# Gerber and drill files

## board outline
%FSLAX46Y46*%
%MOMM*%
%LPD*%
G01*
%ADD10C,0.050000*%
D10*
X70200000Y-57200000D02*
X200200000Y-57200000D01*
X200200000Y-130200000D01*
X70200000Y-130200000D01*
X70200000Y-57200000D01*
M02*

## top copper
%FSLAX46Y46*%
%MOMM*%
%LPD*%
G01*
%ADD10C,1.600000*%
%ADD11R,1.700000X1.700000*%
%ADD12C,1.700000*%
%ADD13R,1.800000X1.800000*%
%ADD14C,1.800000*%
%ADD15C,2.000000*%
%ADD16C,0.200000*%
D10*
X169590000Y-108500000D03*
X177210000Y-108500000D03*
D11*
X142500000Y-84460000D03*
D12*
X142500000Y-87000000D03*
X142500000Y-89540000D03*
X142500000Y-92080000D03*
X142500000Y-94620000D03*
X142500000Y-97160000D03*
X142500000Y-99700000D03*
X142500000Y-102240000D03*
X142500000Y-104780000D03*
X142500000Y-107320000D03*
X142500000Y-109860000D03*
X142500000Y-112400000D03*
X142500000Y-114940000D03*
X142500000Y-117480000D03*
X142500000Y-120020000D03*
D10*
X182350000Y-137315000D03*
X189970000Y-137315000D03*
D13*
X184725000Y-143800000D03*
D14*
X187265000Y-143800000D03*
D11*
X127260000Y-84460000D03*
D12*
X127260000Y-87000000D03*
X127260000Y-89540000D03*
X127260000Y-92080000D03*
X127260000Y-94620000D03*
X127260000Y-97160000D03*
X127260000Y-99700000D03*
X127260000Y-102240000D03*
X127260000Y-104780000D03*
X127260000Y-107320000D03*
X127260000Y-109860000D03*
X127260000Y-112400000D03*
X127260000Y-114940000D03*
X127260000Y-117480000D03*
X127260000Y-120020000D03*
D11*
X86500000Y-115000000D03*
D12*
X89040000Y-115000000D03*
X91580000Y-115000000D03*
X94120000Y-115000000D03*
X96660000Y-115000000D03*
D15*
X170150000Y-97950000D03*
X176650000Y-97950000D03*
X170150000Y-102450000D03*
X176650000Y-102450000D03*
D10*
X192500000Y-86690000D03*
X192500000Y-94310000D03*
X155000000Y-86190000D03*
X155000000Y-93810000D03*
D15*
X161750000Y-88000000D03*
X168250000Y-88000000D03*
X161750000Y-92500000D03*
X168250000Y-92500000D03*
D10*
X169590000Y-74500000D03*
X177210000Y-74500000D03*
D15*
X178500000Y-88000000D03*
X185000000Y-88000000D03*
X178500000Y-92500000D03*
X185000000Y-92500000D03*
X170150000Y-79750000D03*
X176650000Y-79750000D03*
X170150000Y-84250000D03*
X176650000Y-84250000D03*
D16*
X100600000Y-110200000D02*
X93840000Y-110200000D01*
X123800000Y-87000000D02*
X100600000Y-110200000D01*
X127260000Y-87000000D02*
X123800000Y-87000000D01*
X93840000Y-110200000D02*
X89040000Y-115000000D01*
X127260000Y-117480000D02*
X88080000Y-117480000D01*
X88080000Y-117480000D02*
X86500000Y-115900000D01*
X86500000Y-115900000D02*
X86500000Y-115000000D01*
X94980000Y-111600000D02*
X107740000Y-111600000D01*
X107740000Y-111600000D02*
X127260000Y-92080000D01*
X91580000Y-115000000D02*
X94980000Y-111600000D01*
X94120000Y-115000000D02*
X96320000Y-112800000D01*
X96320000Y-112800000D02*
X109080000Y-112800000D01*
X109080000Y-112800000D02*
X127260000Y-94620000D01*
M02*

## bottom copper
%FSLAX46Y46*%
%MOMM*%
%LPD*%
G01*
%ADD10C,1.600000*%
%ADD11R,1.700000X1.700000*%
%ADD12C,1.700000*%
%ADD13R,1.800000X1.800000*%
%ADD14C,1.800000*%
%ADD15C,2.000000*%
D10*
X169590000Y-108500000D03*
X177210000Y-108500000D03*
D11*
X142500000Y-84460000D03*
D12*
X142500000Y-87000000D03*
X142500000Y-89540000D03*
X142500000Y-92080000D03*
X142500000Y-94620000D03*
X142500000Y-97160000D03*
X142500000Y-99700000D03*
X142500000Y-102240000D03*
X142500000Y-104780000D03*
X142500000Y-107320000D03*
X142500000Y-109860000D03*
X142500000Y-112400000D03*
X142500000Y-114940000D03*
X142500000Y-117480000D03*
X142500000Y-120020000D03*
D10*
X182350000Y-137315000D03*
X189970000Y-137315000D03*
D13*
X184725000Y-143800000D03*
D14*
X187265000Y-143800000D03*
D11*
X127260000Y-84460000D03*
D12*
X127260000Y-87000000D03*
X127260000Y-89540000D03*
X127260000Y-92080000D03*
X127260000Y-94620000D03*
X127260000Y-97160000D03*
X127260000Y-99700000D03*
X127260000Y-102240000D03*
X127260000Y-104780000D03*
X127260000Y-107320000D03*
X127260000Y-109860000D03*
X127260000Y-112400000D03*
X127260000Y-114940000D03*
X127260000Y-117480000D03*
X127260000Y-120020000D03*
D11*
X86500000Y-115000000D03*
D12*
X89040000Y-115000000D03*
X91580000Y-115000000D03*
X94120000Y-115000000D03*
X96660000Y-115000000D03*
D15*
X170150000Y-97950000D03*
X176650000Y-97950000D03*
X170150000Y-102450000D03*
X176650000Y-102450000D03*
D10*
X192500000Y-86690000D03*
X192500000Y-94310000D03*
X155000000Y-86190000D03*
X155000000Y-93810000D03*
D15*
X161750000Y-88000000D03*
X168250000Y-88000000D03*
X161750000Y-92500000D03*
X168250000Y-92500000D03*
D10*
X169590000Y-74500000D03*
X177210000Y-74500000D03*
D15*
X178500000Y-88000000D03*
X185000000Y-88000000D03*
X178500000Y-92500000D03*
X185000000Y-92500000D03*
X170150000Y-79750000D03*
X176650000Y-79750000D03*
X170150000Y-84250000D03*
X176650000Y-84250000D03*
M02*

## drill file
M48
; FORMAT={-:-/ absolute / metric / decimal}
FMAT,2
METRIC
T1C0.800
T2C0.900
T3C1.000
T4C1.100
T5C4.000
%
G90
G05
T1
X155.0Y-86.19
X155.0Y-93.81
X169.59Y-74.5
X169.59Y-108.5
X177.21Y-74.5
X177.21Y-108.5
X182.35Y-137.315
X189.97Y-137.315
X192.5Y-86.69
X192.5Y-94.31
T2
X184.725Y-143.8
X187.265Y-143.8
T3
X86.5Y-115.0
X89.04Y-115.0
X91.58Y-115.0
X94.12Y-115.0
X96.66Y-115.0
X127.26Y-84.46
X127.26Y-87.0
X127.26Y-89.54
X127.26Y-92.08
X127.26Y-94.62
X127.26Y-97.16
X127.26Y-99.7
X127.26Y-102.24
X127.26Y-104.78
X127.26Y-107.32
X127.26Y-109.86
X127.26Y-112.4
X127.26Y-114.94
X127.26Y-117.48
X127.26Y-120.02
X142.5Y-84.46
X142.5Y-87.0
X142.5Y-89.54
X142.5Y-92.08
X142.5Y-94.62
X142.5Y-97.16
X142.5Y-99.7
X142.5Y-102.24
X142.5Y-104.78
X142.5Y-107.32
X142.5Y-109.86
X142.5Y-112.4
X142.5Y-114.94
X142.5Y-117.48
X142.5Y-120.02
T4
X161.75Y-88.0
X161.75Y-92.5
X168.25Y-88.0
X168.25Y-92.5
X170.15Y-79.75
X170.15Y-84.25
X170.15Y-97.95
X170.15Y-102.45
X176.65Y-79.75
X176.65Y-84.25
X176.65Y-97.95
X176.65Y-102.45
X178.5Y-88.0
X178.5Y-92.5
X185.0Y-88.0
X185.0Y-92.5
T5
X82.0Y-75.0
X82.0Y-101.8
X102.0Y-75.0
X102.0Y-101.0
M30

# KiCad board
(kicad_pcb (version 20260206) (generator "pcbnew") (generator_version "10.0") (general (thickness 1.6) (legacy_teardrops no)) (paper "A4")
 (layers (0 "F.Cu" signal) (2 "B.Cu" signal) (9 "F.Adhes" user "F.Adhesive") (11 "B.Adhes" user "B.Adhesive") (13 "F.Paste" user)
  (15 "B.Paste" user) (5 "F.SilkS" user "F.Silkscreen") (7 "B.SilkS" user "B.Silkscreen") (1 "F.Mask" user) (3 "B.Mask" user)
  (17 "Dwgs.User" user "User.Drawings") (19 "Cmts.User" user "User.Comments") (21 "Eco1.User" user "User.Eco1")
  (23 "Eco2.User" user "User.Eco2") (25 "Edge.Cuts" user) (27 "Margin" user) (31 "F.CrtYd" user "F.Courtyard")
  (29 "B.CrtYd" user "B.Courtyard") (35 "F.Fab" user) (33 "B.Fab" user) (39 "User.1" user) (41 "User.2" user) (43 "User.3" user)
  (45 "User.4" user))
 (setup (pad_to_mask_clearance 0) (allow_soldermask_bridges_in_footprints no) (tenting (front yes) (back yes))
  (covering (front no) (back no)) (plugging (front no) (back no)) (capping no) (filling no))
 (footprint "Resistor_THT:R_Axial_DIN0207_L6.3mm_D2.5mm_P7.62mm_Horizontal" (layer "F.Cu") (at 169.59 108.5)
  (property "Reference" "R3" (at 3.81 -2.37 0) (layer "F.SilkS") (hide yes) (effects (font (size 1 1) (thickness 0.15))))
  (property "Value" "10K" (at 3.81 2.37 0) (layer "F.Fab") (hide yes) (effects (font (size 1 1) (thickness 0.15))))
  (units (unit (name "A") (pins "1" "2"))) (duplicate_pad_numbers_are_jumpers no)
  (pad "1" thru_hole circle (at 0 0) (size 1.6 1.6) (drill 0.8) (layers "*.Cu" "*.Mask") (remove_unused_layers no) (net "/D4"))
  (pad "2" thru_hole circle (at 7.62 0) (size 1.6 1.6) (drill 0.8) (layers "*.Cu" "*.Mask") (remove_unused_layers no) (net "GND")))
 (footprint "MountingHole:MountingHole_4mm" (layer "F.Cu") (at 102 75)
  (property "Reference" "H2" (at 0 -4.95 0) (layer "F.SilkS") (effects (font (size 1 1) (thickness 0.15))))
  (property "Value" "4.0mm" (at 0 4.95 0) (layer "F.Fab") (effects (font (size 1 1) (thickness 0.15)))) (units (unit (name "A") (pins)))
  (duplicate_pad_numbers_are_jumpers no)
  (pad "" np_thru_hole circle (at 0 0) (size 4 4) (drill 4) (layers "*.Cu" "*.Mask")))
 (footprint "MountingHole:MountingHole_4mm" (layer "F.Cu") (at 82 75)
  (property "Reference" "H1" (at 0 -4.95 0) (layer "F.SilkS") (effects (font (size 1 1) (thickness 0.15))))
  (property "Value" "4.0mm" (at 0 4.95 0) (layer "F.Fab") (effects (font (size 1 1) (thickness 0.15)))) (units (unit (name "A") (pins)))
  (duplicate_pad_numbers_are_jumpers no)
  (pad "" np_thru_hole circle (at 0 0) (size 4 4) (drill 4) (layers "*.Cu" "*.Mask")))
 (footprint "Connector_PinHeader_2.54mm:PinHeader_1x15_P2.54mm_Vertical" (layer "F.Cu") (at 142.5 84.46)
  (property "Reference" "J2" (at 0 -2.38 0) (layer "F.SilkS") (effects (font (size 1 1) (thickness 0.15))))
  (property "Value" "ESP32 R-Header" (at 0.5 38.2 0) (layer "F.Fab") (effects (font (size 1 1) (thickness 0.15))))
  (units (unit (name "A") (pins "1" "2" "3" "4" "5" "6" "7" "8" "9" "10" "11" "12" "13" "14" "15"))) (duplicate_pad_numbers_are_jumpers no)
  (pad "1" thru_hole rect (at 0 0) (size 1.7 1.7) (drill 1) (layers "*.Cu" "*.Mask") (remove_unused_layers no) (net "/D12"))
  (pad "2" thru_hole circle (at 0 2.54) (size 1.7 1.7) (drill 1) (layers "*.Cu" "*.Mask") (remove_unused_layers no) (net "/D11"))
  (pad "3" thru_hole circle (at 0 5.08) (size 1.7 1.7) (drill 1) (layers "*.Cu" "*.Mask") (remove_unused_layers no) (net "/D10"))
  (pad "4" thru_hole circle (at 0 7.62) (size 1.7 1.7) (drill 1) (layers "*.Cu" "*.Mask") (remove_unused_layers no) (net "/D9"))
  (pad "5" thru_hole circle (at 0 10.16) (size 1.7 1.7) (drill 1) (layers "*.Cu" "*.Mask") (remove_unused_layers no) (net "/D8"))
  (pad "6" thru_hole circle (at 0 12.7) (size 1.7 1.7) (drill 1) (layers "*.Cu" "*.Mask") (remove_unused_layers no) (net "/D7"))
  (pad "7" thru_hole circle (at 0 15.24) (size 1.7 1.7) (drill 1) (layers "*.Cu" "*.Mask") (remove_unused_layers no) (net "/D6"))
  (pad "8" thru_hole circle (at 0 17.78) (size 1.7 1.7) (drill 1) (layers "*.Cu" "*.Mask") (remove_unused_layers no) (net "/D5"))
  (pad "9" thru_hole circle (at 0 20.32) (size 1.7 1.7) (drill 1) (layers "*.Cu" "*.Mask") (remove_unused_layers no) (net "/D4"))
  (pad "10" thru_hole circle (at 0 22.86) (size 1.7 1.7) (drill 1) (layers "*.Cu" "*.Mask") (remove_unused_layers no) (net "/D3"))
  (pad "11" thru_hole circle (at 0 25.4) (size 1.7 1.7) (drill 1) (layers "*.Cu" "*.Mask") (remove_unused_layers no) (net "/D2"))
  (pad "12" thru_hole circle (at 0 27.94) (size 1.7 1.7) (drill 1) (layers "*.Cu" "*.Mask") (remove_unused_layers no) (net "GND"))
  (pad "13" thru_hole circle (at 0 30.48) (size 1.7 1.7) (drill 1) (layers "*.Cu" "*.Mask") (remove_unused_layers no) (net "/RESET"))
  (pad "14" thru_hole circle (at 0 33.02) (size 1.7 1.7) (drill 1) (layers "*.Cu" "*.Mask") (remove_unused_layers no) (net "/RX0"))
  (pad "15" thru_hole circle (at 0 35.56) (size 1.7 1.7) (drill 1) (layers "*.Cu" "*.Mask") (remove_unused_layers no) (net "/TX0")))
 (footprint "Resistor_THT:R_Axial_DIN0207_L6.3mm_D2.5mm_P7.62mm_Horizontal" (layer "F.Cu") (at 182.35 137.315)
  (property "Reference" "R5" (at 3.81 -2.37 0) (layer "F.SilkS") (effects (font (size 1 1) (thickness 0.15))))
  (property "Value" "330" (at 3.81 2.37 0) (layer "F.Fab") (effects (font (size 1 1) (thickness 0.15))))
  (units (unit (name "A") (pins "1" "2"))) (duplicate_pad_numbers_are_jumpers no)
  (pad "1" thru_hole circle (at 0 0) (size 1.6 1.6) (drill 0.8) (layers "*.Cu" "*.Mask") (remove_unused_layers no) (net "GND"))
  (pad "2" thru_hole circle (at 7.62 0) (size 1.6 1.6) (drill 0.8) (layers "*.Cu" "*.Mask") (remove_unused_layers no) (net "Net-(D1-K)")))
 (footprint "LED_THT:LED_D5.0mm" (layer "F.Cu") (at 184.725 143.8)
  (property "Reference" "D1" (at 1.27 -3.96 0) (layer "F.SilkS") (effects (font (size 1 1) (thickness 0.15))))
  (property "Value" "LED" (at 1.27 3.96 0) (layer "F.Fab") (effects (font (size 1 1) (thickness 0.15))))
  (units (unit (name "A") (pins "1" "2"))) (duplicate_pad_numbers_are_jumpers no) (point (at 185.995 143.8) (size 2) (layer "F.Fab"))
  (pad "1" thru_hole rect (at 0 0) (size 1.8 1.8) (drill 0.9) (layers "*.Cu" "*.Mask") (remove_unused_layers no) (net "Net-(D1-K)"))
  (pad "2" thru_hole circle (at 2.54 0) (size 1.8 1.8) (drill 0.9) (layers "*.Cu" "*.Mask") (remove_unused_layers no) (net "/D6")))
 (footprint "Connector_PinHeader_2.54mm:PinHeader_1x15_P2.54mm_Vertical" (layer "F.Cu") (at 127.26 84.46)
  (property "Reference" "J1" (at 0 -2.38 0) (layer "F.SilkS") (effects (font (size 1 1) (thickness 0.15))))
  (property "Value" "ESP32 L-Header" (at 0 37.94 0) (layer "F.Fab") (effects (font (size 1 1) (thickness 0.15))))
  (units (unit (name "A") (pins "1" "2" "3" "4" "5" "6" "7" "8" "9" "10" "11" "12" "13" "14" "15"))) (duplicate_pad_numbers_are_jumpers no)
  (pad "1" thru_hole rect (at 0 0) (size 1.7 1.7) (drill 1) (layers "*.Cu" "*.Mask") (remove_unused_layers no) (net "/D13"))
  (pad "2" thru_hole circle (at 0 2.54) (size 1.7 1.7) (drill 1) (layers "*.Cu" "*.Mask") (remove_unused_layers no) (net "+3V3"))
  (pad "3" thru_hole circle (at 0 5.08) (size 1.7 1.7) (drill 1) (layers "*.Cu" "*.Mask") (remove_unused_layers no) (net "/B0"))
  (pad "4" thru_hole circle (at 0 7.62) (size 1.7 1.7) (drill 1) (layers "*.Cu" "*.Mask") (remove_unused_layers no) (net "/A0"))
  (pad "5" thru_hole circle (at 0 10.16) (size 1.7 1.7) (drill 1) (layers "*.Cu" "*.Mask") (remove_unused_layers no) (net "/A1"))
  (pad "6" thru_hole circle (at 0 12.7) (size 1.7 1.7) (drill 1) (layers "*.Cu" "*.Mask") (remove_unused_layers no) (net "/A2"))
  (pad "7" thru_hole circle (at 0 15.24) (size 1.7 1.7) (drill 1) (layers "*.Cu" "*.Mask") (remove_unused_layers no) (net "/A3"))
  (pad "8" thru_hole circle (at 0 17.78) (size 1.7 1.7) (drill 1) (layers "*.Cu" "*.Mask") (remove_unused_layers no) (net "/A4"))
  (pad "9" thru_hole circle (at 0 20.32) (size 1.7 1.7) (drill 1) (layers "*.Cu" "*.Mask") (remove_unused_layers no) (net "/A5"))
  (pad "10" thru_hole circle (at 0 22.86) (size 1.7 1.7) (drill 1) (layers "*.Cu" "*.Mask") (remove_unused_layers no) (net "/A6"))
  (pad "11" thru_hole circle (at 0 25.4) (size 1.7 1.7) (drill 1) (layers "*.Cu" "*.Mask") (remove_unused_layers no) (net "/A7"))
  (pad "12" thru_hole circle (at 0 27.94) (size 1.7 1.7) (drill 1) (layers "*.Cu" "*.Mask") (remove_unused_layers no) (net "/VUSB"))
  (pad "13" thru_hole circle (at 0 30.48) (size 1.7 1.7) (drill 1) (layers "*.Cu" "*.Mask") (remove_unused_layers no) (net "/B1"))
  (pad "14" thru_hole circle (at 0 33.02) (size 1.7 1.7) (drill 1) (layers "*.Cu" "*.Mask") (remove_unused_layers no) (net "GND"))
  (pad "15" thru_hole circle (at 0 35.56) (size 1.7 1.7) (drill 1) (layers "*.Cu" "*.Mask") (remove_unused_layers no) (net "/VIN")))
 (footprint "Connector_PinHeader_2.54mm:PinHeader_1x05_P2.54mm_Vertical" (layer "F.Cu") (at 86.5 115 90)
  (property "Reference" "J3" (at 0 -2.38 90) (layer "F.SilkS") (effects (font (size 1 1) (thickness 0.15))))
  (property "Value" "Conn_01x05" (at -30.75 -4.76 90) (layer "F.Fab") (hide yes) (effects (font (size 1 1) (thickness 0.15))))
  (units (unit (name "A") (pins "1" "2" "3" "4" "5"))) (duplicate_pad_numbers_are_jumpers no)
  (pad "1" thru_hole rect (at 0 0 90) (size 1.7 1.7) (drill 1) (layers "*.Cu" "*.Mask") (remove_unused_layers no) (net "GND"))
  (pad "2" thru_hole circle (at 0 2.54 90) (size 1.7 1.7) (drill 1) (layers "*.Cu" "*.Mask") (remove_unused_layers no) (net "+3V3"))
  (pad "3" thru_hole circle (at 0 5.08 90) (size 1.7 1.7) (drill 1) (layers "*.Cu" "*.Mask") (remove_unused_layers no) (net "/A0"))
  (pad "4" thru_hole circle (at 0 7.62 90) (size 1.7 1.7) (drill 1) (layers "*.Cu" "*.Mask") (remove_unused_layers no) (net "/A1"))
  (pad "5" thru_hole circle (at 0 10.16 90) (size 1.7 1.7) (drill 1) (layers "*.Cu" "*.Mask") (remove_unused_layers no)
   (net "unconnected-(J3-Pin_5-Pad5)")))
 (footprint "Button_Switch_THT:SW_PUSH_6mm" (layer "F.Cu") (at 170.15 97.95)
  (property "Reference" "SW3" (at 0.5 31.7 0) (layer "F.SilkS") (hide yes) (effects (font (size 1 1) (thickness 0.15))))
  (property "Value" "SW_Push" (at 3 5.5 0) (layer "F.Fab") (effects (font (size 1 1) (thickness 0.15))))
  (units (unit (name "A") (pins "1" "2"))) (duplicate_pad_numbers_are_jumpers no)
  (pad "1" thru_hole circle (at 0 0 90) (size 2 2) (drill 1.1) (layers "*.Cu" "*.Mask") (remove_unused_layers no)
   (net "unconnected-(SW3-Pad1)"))
  (pad "1" thru_hole circle (at 6.5 0 90) (size 2 2) (drill 1.1) (layers "*.Cu" "*.Mask") (remove_unused_layers no)
   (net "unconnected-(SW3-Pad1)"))
  (pad "2" thru_hole circle (at 0 4.5 90) (size 2 2) (drill 1.1) (layers "*.Cu" "*.Mask") (remove_unused_layers no) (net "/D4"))
  (pad "2" thru_hole circle (at 6.5 4.5 90) (size 2 2) (drill 1.1) (layers "*.Cu" "*.Mask") (remove_unused_layers no) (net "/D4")))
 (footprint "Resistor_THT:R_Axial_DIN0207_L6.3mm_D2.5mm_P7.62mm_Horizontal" (layer "F.Cu") (at 192.5 86.69 -90)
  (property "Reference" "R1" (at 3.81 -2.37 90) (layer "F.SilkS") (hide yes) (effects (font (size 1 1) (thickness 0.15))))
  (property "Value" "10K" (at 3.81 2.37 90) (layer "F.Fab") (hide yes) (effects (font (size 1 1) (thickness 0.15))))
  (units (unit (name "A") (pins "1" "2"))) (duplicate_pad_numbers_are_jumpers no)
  (pad "1" thru_hole circle (at 0 0 270) (size 1.6 1.6) (drill 0.8) (layers "*.Cu" "*.Mask") (remove_unused_layers no) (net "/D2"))
  (pad "2" thru_hole circle (at 7.62 0 270) (size 1.6 1.6) (drill 0.8) (layers "*.Cu" "*.Mask") (remove_unused_layers no) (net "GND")))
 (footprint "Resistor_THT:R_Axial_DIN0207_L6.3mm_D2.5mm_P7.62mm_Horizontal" (layer "F.Cu") (at 155 86.19 -90)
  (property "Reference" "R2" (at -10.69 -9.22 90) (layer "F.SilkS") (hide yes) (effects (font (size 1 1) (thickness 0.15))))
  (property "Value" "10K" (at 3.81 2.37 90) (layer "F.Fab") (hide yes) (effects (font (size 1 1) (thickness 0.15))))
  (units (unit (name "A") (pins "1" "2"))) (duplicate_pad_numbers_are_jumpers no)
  (pad "1" thru_hole circle (at 0 0 270) (size 1.6 1.6) (drill 0.8) (layers "*.Cu" "*.Mask") (remove_unused_layers no) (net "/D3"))
  (pad "2" thru_hole circle (at 7.62 0 270) (size 1.6 1.6) (drill 0.8) (layers "*.Cu" "*.Mask") (remove_unused_layers no) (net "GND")))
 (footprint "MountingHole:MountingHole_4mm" (layer "F.Cu") (at 82 101.8)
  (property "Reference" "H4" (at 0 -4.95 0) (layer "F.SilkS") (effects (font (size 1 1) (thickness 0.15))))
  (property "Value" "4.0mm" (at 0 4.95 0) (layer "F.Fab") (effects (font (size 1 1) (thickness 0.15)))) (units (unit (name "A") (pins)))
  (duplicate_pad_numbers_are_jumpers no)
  (pad "" np_thru_hole circle (at 0 0) (size 4 4) (drill 4) (layers "*.Cu" "*.Mask")))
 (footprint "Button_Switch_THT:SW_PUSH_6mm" (layer "F.Cu") (at 161.75 88)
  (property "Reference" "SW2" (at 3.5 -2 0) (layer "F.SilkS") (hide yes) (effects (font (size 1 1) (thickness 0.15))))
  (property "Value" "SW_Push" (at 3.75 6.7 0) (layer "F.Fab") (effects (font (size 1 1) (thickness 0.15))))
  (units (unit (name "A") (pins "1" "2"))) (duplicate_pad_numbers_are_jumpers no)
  (pad "1" thru_hole circle (at 0 0 90) (size 2 2) (drill 1.1) (layers "*.Cu" "*.Mask") (remove_unused_layers no) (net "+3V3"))
  (pad "1" thru_hole circle (at 6.5 0 90) (size 2 2) (drill 1.1) (layers "*.Cu" "*.Mask") (remove_unused_layers no) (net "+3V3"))
  (pad "2" thru_hole circle (at 0 4.5 90) (size 2 2) (drill 1.1) (layers "*.Cu" "*.Mask") (remove_unused_layers no) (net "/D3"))
  (pad "2" thru_hole circle (at 6.5 4.5 90) (size 2 2) (drill 1.1) (layers "*.Cu" "*.Mask") (remove_unused_layers no) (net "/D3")))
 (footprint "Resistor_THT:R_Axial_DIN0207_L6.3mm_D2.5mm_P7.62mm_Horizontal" (layer "F.Cu") (at 169.59 74.5)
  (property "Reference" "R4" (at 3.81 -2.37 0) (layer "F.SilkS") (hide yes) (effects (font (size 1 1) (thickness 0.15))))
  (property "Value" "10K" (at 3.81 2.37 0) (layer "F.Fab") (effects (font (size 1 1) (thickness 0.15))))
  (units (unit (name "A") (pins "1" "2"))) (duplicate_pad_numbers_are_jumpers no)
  (pad "1" thru_hole circle (at 0 0) (size 1.6 1.6) (drill 0.8) (layers "*.Cu" "*.Mask") (remove_unused_layers no) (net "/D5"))
  (pad "2" thru_hole circle (at 7.62 0) (size 1.6 1.6) (drill 0.8) (layers "*.Cu" "*.Mask") (remove_unused_layers no) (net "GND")))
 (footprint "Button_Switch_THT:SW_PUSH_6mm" (layer "F.Cu") (at 178.5 88)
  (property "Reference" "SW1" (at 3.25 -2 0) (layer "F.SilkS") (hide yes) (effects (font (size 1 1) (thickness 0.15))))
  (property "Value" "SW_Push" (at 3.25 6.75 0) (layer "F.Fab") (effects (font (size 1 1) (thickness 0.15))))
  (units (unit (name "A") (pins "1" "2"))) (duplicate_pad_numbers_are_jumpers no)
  (pad "1" thru_hole circle (at 0 0 90) (size 2 2) (drill 1.1) (layers "*.Cu" "*.Mask") (remove_unused_layers no) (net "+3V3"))
  (pad "1" thru_hole circle (at 6.5 0 90) (size 2 2) (drill 1.1) (layers "*.Cu" "*.Mask") (remove_unused_layers no) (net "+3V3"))
  (pad "2" thru_hole circle (at 0 4.5 90) (size 2 2) (drill 1.1) (layers "*.Cu" "*.Mask") (remove_unused_layers no) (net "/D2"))
  (pad "2" thru_hole circle (at 6.5 4.5 90) (size 2 2) (drill 1.1) (layers "*.Cu" "*.Mask") (remove_unused_layers no) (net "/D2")))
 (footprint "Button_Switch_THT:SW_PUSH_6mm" (layer "F.Cu") (at 170.15 79.75)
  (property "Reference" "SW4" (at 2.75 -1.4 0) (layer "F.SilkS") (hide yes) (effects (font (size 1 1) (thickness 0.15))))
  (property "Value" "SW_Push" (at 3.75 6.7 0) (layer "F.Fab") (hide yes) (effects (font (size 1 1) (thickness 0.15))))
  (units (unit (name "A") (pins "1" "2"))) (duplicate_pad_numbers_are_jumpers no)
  (pad "1" thru_hole circle (at 0 0 90) (size 2 2) (drill 1.1) (layers "*.Cu" "*.Mask") (remove_unused_layers no)
   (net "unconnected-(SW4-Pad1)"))
  (pad "1" thru_hole circle (at 6.5 0 90) (size 2 2) (drill 1.1) (layers "*.Cu" "*.Mask") (remove_unused_layers no)
   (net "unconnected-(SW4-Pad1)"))
  (pad "2" thru_hole circle (at 0 4.5 90) (size 2 2) (drill 1.1) (layers "*.Cu" "*.Mask") (remove_unused_layers no) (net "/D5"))
  (pad "2" thru_hole circle (at 6.5 4.5 90) (size 2 2) (drill 1.1) (layers "*.Cu" "*.Mask") (remove_unused_layers no) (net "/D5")))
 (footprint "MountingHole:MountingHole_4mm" (layer "F.Cu") (at 102 101)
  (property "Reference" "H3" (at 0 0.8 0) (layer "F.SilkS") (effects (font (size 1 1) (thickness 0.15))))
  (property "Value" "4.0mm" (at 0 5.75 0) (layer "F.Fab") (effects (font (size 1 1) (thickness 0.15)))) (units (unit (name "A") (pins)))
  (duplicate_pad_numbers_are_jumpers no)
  (pad "" np_thru_hole circle (at 0 0) (size 4 4) (drill 4) (layers "*.Cu" "*.Mask")))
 (gr_rect (start 70.2 57.2) (end 200.2 130.2) (stroke (width 0.05) (type default)) (fill no) (layer "Edge.Cuts"))
 (segment (start 100.6 110.2) (end 93.84 110.2) (width 0.2) (layer "F.Cu") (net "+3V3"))
 (segment (start 123.8 87) (end 100.6 110.2) (width 0.2) (layer "F.Cu") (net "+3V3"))
 (segment (start 127.26 87) (end 123.8 87) (width 0.2) (layer "F.Cu") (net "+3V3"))
 (segment (start 93.84 110.2) (end 89.04 115) (width 0.2) (layer "F.Cu") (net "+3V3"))
 (segment (start 127.26 117.48) (end 88.08 117.48) (width 0.2) (layer "F.Cu") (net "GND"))
 (segment (start 88.08 117.48) (end 86.5 115.9) (width 0.2) (layer "F.Cu") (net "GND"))
 (segment (start 86.5 115.9) (end 86.5 115) (width 0.2) (layer "F.Cu") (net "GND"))
 (segment (start 94.98 111.6) (end 107.74 111.6) (width 0.2) (layer "F.Cu") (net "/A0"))
 (segment (start 107.74 111.6) (end 127.26 92.08) (width 0.2) (layer "F.Cu") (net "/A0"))
 (segment (start 91.58 115) (end 94.98 111.6) (width 0.2) (layer "F.Cu") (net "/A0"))
 (segment (start 94.12 115) (end 96.32 112.8) (width 0.2) (layer "F.Cu") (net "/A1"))
 (segment (start 96.32 112.8) (end 109.08 112.8) (width 0.2) (layer "F.Cu") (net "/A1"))
 (segment (start 109.08 112.8) (end 127.26 94.62) (width 0.2) (layer "F.Cu") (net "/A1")))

